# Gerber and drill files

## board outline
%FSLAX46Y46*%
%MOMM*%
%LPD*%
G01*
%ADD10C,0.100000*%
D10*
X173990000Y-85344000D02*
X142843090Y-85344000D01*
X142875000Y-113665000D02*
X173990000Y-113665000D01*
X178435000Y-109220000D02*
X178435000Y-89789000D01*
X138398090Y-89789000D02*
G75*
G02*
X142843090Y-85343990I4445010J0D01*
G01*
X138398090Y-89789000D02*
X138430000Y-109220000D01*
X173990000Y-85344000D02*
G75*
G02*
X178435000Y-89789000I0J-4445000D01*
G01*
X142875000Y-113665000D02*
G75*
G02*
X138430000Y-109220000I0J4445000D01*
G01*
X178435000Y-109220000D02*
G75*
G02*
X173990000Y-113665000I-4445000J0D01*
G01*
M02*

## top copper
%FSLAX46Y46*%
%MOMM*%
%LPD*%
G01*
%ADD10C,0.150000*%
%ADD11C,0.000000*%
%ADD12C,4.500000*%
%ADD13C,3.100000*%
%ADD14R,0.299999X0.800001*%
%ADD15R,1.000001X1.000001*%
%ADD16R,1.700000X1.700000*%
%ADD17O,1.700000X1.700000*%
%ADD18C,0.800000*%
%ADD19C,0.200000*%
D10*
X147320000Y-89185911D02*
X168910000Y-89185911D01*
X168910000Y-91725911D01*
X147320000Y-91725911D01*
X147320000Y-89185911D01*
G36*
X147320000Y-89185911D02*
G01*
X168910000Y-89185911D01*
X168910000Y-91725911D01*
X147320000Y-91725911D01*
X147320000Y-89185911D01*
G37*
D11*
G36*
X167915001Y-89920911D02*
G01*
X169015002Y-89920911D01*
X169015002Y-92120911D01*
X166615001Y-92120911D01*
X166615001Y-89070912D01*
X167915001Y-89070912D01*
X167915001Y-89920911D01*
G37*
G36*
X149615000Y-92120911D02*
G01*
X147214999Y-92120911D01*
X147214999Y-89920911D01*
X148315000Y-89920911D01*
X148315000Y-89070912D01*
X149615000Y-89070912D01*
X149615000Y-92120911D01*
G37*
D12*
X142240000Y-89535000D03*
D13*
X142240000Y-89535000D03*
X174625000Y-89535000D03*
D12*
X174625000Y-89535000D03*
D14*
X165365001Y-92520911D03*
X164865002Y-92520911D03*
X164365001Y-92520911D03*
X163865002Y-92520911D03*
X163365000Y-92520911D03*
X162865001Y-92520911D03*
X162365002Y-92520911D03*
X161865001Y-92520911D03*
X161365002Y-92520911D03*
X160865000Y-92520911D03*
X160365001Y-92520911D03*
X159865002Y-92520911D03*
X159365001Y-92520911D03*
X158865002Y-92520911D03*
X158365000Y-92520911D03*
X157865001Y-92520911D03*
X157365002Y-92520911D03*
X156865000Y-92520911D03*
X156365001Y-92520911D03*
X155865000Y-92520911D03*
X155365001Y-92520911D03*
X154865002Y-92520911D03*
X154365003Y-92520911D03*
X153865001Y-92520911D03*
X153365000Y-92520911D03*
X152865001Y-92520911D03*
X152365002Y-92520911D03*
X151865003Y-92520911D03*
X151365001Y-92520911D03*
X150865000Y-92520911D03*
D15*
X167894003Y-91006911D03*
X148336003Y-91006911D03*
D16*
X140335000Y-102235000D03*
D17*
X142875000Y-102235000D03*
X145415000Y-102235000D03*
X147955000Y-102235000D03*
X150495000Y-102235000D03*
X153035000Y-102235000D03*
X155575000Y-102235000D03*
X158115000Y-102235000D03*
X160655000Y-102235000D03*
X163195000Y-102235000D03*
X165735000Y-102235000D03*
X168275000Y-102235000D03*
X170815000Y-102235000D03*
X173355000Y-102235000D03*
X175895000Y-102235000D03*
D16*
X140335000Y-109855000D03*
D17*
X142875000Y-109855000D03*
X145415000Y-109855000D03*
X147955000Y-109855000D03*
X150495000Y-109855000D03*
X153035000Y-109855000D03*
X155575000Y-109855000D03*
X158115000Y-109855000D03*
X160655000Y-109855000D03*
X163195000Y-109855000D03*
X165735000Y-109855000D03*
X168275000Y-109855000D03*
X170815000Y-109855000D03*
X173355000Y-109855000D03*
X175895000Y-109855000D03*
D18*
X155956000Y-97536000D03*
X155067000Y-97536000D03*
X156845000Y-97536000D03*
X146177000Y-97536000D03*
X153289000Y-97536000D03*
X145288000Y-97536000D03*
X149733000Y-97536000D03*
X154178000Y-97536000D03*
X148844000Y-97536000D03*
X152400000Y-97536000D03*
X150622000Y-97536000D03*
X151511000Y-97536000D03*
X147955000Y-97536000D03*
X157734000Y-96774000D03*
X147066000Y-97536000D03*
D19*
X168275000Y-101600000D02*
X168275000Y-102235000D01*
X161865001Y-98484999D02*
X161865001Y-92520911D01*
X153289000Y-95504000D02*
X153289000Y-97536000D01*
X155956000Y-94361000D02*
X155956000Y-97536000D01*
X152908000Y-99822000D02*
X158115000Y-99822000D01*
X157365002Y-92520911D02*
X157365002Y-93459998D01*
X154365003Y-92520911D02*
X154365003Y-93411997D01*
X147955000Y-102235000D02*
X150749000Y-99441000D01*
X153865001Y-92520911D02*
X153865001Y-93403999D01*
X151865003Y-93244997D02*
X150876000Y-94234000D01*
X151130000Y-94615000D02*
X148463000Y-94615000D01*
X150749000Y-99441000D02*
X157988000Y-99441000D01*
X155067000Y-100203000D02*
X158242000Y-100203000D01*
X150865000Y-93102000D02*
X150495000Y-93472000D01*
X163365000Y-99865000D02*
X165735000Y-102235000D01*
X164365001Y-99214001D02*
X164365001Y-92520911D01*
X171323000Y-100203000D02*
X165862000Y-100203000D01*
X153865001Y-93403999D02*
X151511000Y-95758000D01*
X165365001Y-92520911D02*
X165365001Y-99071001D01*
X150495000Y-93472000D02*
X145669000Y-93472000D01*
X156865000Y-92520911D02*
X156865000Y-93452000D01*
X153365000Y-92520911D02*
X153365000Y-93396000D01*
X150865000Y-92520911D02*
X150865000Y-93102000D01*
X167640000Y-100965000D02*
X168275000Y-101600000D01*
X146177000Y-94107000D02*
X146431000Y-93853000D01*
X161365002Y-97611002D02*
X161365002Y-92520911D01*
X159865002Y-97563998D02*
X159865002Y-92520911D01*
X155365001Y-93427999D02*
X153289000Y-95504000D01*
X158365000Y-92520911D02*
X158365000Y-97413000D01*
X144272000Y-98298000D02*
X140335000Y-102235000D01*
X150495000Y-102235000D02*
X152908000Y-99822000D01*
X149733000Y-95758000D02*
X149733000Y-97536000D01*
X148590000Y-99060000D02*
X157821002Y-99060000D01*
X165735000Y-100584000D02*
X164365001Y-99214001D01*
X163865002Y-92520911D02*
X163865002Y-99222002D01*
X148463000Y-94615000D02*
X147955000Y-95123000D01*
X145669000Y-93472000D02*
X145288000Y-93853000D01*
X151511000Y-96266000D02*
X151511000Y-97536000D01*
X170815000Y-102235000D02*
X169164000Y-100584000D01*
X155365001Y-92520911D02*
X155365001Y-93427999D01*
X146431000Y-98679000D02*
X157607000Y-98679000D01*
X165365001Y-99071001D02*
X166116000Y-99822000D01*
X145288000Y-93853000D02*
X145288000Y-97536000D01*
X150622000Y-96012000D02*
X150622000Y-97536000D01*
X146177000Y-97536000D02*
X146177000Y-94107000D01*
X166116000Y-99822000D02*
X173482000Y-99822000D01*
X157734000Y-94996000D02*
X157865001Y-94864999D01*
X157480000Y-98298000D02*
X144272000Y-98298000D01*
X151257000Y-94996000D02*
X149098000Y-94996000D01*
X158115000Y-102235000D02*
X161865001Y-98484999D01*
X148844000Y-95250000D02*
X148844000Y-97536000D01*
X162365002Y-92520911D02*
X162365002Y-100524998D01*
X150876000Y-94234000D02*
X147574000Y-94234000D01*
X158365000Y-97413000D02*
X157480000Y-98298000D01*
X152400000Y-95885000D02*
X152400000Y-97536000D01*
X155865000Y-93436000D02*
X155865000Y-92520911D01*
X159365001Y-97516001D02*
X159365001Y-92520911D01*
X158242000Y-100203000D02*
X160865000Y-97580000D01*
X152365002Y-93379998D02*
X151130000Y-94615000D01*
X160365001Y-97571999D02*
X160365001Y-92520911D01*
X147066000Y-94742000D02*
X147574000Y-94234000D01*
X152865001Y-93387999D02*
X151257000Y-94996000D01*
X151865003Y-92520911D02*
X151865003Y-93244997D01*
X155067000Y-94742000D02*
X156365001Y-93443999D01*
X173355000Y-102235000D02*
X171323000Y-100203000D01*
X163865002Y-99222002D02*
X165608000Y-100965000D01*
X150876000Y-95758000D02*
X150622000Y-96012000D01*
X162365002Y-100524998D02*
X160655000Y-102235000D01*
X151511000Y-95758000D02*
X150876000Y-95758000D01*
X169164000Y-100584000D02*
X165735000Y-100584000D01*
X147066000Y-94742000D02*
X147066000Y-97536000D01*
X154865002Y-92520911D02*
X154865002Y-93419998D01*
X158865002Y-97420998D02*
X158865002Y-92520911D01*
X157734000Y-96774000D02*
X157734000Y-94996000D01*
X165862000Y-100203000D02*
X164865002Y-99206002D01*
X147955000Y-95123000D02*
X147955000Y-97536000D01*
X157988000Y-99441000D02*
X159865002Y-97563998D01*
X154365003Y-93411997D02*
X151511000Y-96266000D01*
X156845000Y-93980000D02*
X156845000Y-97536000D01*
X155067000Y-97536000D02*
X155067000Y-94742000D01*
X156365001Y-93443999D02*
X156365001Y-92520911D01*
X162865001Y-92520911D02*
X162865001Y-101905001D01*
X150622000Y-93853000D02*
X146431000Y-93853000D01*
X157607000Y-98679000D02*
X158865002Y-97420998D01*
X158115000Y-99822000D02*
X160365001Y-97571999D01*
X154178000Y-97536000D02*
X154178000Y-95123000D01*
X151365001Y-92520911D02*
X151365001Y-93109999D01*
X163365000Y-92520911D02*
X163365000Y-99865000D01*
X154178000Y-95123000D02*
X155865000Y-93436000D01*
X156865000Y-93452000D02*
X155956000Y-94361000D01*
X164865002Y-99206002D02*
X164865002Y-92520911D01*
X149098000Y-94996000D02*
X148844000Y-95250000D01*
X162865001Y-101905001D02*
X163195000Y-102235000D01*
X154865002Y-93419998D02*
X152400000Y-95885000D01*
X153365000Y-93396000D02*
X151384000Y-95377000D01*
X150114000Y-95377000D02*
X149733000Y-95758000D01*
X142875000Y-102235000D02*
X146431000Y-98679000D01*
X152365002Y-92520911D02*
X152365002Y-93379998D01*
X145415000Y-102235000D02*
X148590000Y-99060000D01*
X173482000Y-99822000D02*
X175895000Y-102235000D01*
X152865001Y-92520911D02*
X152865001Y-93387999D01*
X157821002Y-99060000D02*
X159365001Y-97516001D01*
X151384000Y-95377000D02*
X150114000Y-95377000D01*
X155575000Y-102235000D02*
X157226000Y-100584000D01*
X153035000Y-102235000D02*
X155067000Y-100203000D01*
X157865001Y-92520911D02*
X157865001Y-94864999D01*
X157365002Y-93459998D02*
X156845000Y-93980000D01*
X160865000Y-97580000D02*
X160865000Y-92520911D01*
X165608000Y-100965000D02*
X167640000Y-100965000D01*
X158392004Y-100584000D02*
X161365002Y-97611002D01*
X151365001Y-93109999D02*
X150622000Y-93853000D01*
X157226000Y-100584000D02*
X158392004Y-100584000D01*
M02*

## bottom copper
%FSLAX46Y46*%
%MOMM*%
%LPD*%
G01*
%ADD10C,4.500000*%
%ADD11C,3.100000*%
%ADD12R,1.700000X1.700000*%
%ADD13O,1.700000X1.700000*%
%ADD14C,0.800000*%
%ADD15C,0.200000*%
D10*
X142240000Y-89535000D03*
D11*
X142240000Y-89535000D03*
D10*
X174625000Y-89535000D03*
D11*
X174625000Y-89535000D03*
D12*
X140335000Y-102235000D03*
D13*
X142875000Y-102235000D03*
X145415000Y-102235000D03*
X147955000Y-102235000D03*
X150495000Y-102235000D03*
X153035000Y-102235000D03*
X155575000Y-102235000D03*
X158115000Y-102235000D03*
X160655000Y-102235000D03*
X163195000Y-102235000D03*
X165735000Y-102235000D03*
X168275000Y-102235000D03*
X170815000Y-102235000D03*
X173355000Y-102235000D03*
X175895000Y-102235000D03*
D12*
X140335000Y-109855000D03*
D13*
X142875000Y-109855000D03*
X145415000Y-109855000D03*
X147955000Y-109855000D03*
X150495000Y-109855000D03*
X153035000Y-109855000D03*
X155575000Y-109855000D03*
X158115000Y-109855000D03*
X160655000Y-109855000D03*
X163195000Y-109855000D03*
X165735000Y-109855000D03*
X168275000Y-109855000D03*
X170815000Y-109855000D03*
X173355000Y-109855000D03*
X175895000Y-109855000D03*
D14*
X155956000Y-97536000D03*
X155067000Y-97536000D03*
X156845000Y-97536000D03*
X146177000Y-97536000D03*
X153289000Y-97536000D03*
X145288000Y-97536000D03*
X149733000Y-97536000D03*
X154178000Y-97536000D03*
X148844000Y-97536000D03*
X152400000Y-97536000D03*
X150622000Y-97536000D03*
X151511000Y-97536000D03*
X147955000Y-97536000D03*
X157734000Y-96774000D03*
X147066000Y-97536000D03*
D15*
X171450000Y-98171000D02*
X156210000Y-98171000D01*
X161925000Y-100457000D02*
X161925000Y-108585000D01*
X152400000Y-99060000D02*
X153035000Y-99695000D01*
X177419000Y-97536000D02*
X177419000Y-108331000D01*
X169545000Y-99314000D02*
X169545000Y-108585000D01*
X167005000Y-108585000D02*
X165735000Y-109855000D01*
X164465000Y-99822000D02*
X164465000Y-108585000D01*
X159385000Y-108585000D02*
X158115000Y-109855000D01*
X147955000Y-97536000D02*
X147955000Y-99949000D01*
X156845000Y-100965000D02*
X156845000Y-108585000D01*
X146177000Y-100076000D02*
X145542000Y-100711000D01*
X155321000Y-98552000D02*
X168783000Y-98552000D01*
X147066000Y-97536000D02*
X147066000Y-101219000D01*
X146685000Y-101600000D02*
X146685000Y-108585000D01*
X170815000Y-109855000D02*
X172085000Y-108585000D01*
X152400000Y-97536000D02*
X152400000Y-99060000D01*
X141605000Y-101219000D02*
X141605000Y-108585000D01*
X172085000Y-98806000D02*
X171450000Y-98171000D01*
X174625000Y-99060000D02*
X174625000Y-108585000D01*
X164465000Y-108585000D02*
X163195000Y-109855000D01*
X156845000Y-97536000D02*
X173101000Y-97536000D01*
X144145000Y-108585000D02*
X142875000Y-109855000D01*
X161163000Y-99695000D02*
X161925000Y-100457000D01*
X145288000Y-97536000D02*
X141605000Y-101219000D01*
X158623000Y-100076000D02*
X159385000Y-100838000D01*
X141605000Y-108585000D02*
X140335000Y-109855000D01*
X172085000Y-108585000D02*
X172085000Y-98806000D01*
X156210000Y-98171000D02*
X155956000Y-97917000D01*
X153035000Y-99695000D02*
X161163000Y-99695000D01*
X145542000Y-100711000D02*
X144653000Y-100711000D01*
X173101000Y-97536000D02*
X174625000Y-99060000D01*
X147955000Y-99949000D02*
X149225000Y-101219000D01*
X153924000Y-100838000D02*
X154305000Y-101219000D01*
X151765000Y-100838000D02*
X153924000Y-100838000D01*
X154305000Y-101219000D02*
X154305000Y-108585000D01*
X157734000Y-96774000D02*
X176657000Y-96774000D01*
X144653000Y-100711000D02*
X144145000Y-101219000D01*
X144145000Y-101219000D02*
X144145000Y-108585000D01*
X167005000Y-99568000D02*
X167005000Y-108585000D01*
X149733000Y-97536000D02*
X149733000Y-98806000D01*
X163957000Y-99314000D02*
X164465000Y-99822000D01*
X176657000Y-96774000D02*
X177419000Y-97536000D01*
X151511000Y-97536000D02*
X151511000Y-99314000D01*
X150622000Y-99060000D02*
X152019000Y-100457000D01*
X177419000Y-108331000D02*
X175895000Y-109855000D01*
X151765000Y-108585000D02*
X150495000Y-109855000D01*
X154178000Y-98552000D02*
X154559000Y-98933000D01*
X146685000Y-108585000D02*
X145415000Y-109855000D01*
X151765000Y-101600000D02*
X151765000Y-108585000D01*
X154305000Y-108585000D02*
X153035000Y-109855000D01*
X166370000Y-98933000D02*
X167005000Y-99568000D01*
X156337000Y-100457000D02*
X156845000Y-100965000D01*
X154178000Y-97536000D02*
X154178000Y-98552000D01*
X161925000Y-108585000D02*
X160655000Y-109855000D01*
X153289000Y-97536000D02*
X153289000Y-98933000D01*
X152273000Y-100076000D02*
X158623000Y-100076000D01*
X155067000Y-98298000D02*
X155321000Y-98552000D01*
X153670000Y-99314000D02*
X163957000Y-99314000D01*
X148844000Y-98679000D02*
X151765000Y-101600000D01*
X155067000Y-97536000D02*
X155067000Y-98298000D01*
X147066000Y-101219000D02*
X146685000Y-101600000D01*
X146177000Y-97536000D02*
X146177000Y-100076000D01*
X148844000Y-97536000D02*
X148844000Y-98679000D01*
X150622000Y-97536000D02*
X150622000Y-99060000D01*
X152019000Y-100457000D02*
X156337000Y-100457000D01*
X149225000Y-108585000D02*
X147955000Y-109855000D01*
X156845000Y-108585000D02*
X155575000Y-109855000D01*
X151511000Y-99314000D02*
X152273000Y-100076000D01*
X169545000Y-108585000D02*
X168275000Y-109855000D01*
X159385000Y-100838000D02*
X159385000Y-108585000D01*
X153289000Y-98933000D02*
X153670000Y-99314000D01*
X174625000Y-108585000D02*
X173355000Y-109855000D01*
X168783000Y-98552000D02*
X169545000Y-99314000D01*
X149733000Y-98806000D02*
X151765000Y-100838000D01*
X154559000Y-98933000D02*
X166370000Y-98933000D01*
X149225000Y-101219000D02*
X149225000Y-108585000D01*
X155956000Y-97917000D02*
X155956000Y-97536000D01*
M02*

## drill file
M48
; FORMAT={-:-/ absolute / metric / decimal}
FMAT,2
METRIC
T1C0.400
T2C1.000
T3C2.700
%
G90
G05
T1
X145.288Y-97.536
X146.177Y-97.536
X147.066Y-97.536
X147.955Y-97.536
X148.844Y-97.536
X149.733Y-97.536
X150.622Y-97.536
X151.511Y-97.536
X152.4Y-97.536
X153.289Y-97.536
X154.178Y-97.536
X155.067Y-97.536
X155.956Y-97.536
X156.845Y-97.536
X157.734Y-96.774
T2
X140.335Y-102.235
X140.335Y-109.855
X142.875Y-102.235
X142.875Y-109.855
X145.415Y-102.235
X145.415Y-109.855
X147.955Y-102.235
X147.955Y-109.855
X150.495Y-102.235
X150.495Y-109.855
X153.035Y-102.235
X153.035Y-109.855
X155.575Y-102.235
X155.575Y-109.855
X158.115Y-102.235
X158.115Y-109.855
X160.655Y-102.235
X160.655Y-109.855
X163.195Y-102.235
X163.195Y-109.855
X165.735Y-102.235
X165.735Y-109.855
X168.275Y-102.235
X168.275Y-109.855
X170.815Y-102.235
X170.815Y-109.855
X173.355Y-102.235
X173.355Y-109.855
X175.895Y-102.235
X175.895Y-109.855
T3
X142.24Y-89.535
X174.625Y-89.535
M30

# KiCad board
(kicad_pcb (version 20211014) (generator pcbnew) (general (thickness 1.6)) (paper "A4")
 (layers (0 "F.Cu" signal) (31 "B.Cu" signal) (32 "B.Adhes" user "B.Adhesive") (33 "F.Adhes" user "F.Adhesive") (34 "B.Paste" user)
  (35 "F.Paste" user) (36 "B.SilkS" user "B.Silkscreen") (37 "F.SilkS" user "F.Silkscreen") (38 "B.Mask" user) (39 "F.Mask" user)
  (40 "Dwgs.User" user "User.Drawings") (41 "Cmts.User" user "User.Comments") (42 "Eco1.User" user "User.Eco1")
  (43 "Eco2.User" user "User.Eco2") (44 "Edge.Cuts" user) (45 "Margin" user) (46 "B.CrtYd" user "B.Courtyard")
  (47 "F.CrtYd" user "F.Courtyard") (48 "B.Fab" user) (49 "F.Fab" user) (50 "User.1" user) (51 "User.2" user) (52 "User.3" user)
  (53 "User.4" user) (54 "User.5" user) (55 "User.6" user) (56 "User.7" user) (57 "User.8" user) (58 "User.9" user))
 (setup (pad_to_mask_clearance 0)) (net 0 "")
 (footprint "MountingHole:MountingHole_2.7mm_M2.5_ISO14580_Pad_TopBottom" (layer "F.Cu") (at 142.24 89.535)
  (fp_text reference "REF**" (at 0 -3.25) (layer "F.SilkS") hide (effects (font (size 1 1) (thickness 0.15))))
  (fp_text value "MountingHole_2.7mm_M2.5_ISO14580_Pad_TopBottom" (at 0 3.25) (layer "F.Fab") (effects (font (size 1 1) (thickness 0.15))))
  (pad "1" connect circle (at 0 0) (size 4.5 4.5) (layers "B.Cu" "B.Mask"))
  (pad "1" connect circle (at 0 0) (size 4.5 4.5) (layers "F.Cu" "F.Mask"))
  (pad "1" thru_hole circle (at 0 0) (size 3.1 3.1) (drill 2.7) (layers *.Cu *.Mask)))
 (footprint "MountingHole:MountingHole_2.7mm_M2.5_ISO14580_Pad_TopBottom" (layer "F.Cu") (at 174.625 89.535)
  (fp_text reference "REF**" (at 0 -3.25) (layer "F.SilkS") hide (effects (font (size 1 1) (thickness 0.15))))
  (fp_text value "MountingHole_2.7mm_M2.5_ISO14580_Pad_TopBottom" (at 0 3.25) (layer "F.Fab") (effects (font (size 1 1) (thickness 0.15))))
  (pad "1" connect circle (at 0 0) (size 4.5 4.5) (layers "B.Cu" "B.Mask"))
  (pad "1" thru_hole circle (at 0 0) (size 3.1 3.1) (drill 2.7) (layers *.Cu *.Mask))
  (pad "1" connect circle (at 0 0) (size 4.5 4.5) (layers "F.Cu" "F.Mask")))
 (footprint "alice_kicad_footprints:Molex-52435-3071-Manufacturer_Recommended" (layer "F.Cu") (at 158.115003 91.758908 180)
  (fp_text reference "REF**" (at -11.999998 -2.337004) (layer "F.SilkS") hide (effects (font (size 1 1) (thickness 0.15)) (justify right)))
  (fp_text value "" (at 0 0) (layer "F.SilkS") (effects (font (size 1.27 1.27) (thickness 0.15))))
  (fp_poly
   (pts (xy -8.499998 -0.362003) (xy -10.899999 -0.362003) (xy -10.899999 1.837997) (xy -9.799998 1.837997) (xy -9.799998 2.687996)
    (xy -8.499998 2.687996))
   (layer "F.Cu") (width 0) (fill solid))
  (fp_poly
   (pts (xy 8.500003 -0.362003) (xy 10.900004 -0.362003) (xy 10.900004 1.837997) (xy 9.800003 1.837997) (xy 9.800003 2.687996)
    (xy 8.500003 2.687996))
   (layer "F.Cu") (width 0) (fill solid))
  (pad "1" smd rect locked (at -7.249998 -0.762003) (size 0.299999 0.800001) (layers "F.Cu" "F.Paste" "F.Mask"))
  (pad "2" smd rect locked (at -6.749999 -0.762003) (size 0.299999 0.800001) (layers "F.Cu" "F.Paste" "F.Mask"))
  (pad "3" smd rect locked (at -6.249998 -0.762003) (size 0.299999 0.800001) (layers "F.Cu" "F.Paste" "F.Mask"))
  (pad "4" smd rect locked (at -5.749999 -0.762003) (size 0.299999 0.800001) (layers "F.Cu" "F.Paste" "F.Mask"))
  (pad "5" smd rect locked (at -5.249997 -0.762003) (size 0.299999 0.800001) (layers "F.Cu" "F.Paste" "F.Mask"))
  (pad "6" smd rect locked (at -4.749998 -0.762003) (size 0.299999 0.800001) (layers "F.Cu" "F.Paste" "F.Mask"))
  (pad "7" smd rect locked (at -4.249999 -0.762003) (size 0.299999 0.800001) (layers "F.Cu" "F.Paste" "F.Mask"))
  (pad "8" smd rect locked (at -3.749998 -0.762003) (size 0.299999 0.800001) (layers "F.Cu" "F.Paste" "F.Mask"))
  (pad "9" smd rect locked (at -3.249999 -0.762003) (size 0.299999 0.800001) (layers "F.Cu" "F.Paste" "F.Mask"))
  (pad "10" smd rect locked (at -2.749997 -0.762003) (size 0.299999 0.800001) (layers "F.Cu" "F.Paste" "F.Mask"))
  (pad "11" smd rect locked (at -2.249998 -0.762003) (size 0.299999 0.800001) (layers "F.Cu" "F.Paste" "F.Mask"))
  (pad "12" smd rect locked (at -1.749999 -0.762003) (size 0.299999 0.800001) (layers "F.Cu" "F.Paste" "F.Mask"))
  (pad "13" smd rect locked (at -1.249998 -0.762003) (size 0.299999 0.800001) (layers "F.Cu" "F.Paste" "F.Mask"))
  (pad "14" smd rect locked (at -0.749999 -0.762003) (size 0.299999 0.800001) (layers "F.Cu" "F.Paste" "F.Mask"))
  (pad "15" smd rect locked (at -0.249997 -0.762003) (size 0.299999 0.800001) (layers "F.Cu" "F.Paste" "F.Mask"))
  (pad "16" smd rect locked (at 0.250002 -0.762003) (size 0.299999 0.800001) (layers "F.Cu" "F.Paste" "F.Mask"))
  (pad "17" smd rect locked (at 0.750001 -0.762003) (size 0.299999 0.800001) (layers "F.Cu" "F.Paste" "F.Mask"))
  (pad "18" smd rect locked (at 1.250003 -0.762003) (size 0.299999 0.800001) (layers "F.Cu" "F.Paste" "F.Mask"))
  (pad "19" smd rect locked (at 1.750002 -0.762003) (size 0.299999 0.800001) (layers "F.Cu" "F.Paste" "F.Mask"))
  (pad "20" smd rect locked (at 2.250003 -0.762003) (size 0.299999 0.800001) (layers "F.Cu" "F.Paste" "F.Mask"))
  (pad "21" smd rect locked (at 2.750002 -0.762003) (size 0.299999 0.800001) (layers "F.Cu" "F.Paste" "F.Mask"))
  (pad "22" smd rect locked (at 3.250001 -0.762003) (size 0.299999 0.800001) (layers "F.Cu" "F.Paste" "F.Mask"))
  (pad "23" smd rect locked (at 3.75 -0.762003) (size 0.299999 0.800001) (layers "F.Cu" "F.Paste" "F.Mask"))
  (pad "24" smd rect locked (at 4.250002 -0.762003) (size 0.299999 0.800001) (layers "F.Cu" "F.Paste" "F.Mask"))
  (pad "25" smd rect locked (at 4.750003 -0.762003) (size 0.299999 0.800001) (layers "F.Cu" "F.Paste" "F.Mask"))
  (pad "26" smd rect locked (at 5.250002 -0.762003) (size 0.299999 0.800001) (layers "F.Cu" "F.Paste" "F.Mask"))
  (pad "27" smd rect locked (at 5.750001 -0.762003) (size 0.299999 0.800001) (layers "F.Cu" "F.Paste" "F.Mask"))
  (pad "28" smd rect locked (at 6.25 -0.762003) (size 0.299999 0.800001) (layers "F.Cu" "F.Paste" "F.Mask"))
  (pad "29" smd rect locked (at 6.750002 -0.762003) (size 0.299999 0.800001) (layers "F.Cu" "F.Paste" "F.Mask"))
  (pad "30" smd rect locked (at 7.250003 -0.762003) (size 0.299999 0.800001) (layers "F.Cu" "F.Paste" "F.Mask"))
  (pad "MP1" smd rect locked (at -9.779 0.751997) (size 1.000001 1.000001) (layers "F.Cu" "F.Paste" "F.Mask"))
  (pad "MP2" smd rect locked (at 9.779 0.751997) (size 1.000001 1.000001) (layers "F.Cu" "F.Paste" "F.Mask")))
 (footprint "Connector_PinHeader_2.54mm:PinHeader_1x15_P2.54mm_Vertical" (layer "F.Cu") (at 140.335 102.235 90)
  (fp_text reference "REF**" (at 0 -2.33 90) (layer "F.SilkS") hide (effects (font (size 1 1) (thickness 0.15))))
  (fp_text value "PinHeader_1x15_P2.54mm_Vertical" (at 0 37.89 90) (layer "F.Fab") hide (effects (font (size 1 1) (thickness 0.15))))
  (pad "1" thru_hole rect (at 0 0 90) (size 1.7 1.7) (drill 1) (layers *.Cu *.Mask))
  (pad "2" thru_hole oval (at 0 2.54 90) (size 1.7 1.7) (drill 1) (layers *.Cu *.Mask))
  (pad "3" thru_hole oval (at 0 5.08 90) (size 1.7 1.7) (drill 1) (layers *.Cu *.Mask))
  (pad "4" thru_hole oval (at 0 7.62 90) (size 1.7 1.7) (drill 1) (layers *.Cu *.Mask))
  (pad "5" thru_hole oval (at 0 10.16 90) (size 1.7 1.7) (drill 1) (layers *.Cu *.Mask))
  (pad "6" thru_hole oval (at 0 12.7 90) (size 1.7 1.7) (drill 1) (layers *.Cu *.Mask))
  (pad "7" thru_hole oval (at 0 15.24 90) (size 1.7 1.7) (drill 1) (layers *.Cu *.Mask))
  (pad "8" thru_hole oval (at 0 17.78 90) (size 1.7 1.7) (drill 1) (layers *.Cu *.Mask))
  (pad "9" thru_hole oval (at 0 20.32 90) (size 1.7 1.7) (drill 1) (layers *.Cu *.Mask))
  (pad "10" thru_hole oval (at 0 22.86 90) (size 1.7 1.7) (drill 1) (layers *.Cu *.Mask))
  (pad "11" thru_hole oval (at 0 25.4 90) (size 1.7 1.7) (drill 1) (layers *.Cu *.Mask))
  (pad "12" thru_hole oval (at 0 27.94 90) (size 1.7 1.7) (drill 1) (layers *.Cu *.Mask))
  (pad "13" thru_hole oval (at 0 30.48 90) (size 1.7 1.7) (drill 1) (layers *.Cu *.Mask))
  (pad "14" thru_hole oval (at 0 33.02 90) (size 1.7 1.7) (drill 1) (layers *.Cu *.Mask))
  (pad "15" thru_hole oval (at 0 35.56 90) (size 1.7 1.7) (drill 1) (layers *.Cu *.Mask)))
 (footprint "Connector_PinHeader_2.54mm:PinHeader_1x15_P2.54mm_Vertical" (layer "F.Cu") (at 140.335 109.855 90)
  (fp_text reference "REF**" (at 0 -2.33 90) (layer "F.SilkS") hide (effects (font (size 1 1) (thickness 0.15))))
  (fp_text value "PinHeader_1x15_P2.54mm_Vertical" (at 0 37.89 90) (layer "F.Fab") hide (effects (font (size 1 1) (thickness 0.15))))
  (pad "1" thru_hole rect (at 0 0 90) (size 1.7 1.7) (drill 1) (layers *.Cu *.Mask))
  (pad "2" thru_hole oval (at 0 2.54 90) (size 1.7 1.7) (drill 1) (layers *.Cu *.Mask))
  (pad "3" thru_hole oval (at 0 5.08 90) (size 1.7 1.7) (drill 1) (layers *.Cu *.Mask))
  (pad "4" thru_hole oval (at 0 7.62 90) (size 1.7 1.7) (drill 1) (layers *.Cu *.Mask))
  (pad "5" thru_hole oval (at 0 10.16 90) (size 1.7 1.7) (drill 1) (layers *.Cu *.Mask))
  (pad "6" thru_hole oval (at 0 12.7 90) (size 1.7 1.7) (drill 1) (layers *.Cu *.Mask))
  (pad "7" thru_hole oval (at 0 15.24 90) (size 1.7 1.7) (drill 1) (layers *.Cu *.Mask))
  (pad "8" thru_hole oval (at 0 17.78 90) (size 1.7 1.7) (drill 1) (layers *.Cu *.Mask))
  (pad "9" thru_hole oval (at 0 20.32 90) (size 1.7 1.7) (drill 1) (layers *.Cu *.Mask))
  (pad "10" thru_hole oval (at 0 22.86 90) (size 1.7 1.7) (drill 1) (layers *.Cu *.Mask))
  (pad "11" thru_hole oval (at 0 25.4 90) (size 1.7 1.7) (drill 1) (layers *.Cu *.Mask))
  (pad "12" thru_hole oval (at 0 27.94 90) (size 1.7 1.7) (drill 1) (layers *.Cu *.Mask))
  (pad "13" thru_hole oval (at 0 30.48 90) (size 1.7 1.7) (drill 1) (layers *.Cu *.Mask))
  (pad "14" thru_hole oval (at 0 33.02 90) (size 1.7 1.7) (drill 1) (layers *.Cu *.Mask))
  (pad "15" thru_hole oval (at 0 35.56 90) (size 1.7 1.7) (drill 1) (layers *.Cu *.Mask)))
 (gr_rect (start 147.32 91.725911) (end 168.91 89.185911) (layer "F.Cu") (width 0.15) (fill solid))
 (gr_line (start 173.99 85.344) (end 142.84309 85.344) (layer "Edge.Cuts") (width 0.1))
 (gr_line (start 142.875 113.665) (end 173.99 113.665) (layer "Edge.Cuts") (width 0.1))
 (gr_line (start 178.435 109.22) (end 178.435 89.789) (layer "Edge.Cuts") (width 0.1))
 (gr_arc (start 138.39809 89.789) (mid 139.7 86.64591) (end 142.84309 85.344) (layer "Edge.Cuts") (width 0.1))
 (gr_line (start 138.39809 89.789) (end 138.43 109.22) (layer "Edge.Cuts") (width 0.1))
 (gr_arc (start 173.99 85.344) (mid 177.13309 86.64591) (end 178.435 89.789) (layer "Edge.Cuts") (width 0.1))
 (gr_arc (start 142.875 113.665) (mid 139.73191 112.36309) (end 138.43 109.22) (layer "Edge.Cuts") (width 0.1))
 (gr_arc (start 178.435 109.22) (mid 177.13309 112.36309) (end 173.99 113.665) (layer "Edge.Cuts") (width 0.1))
 (segment (start 168.275 101.6) (end 168.275 102.235) (width 0.2) (layer "F.Cu") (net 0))
 (segment (start 161.865001 98.484999) (end 161.865001 92.520911) (width 0.2) (layer "F.Cu") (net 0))
 (segment (start 153.289 95.504) (end 153.289 97.536) (width 0.2) (layer "F.Cu") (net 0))
 (segment (start 155.956 94.361) (end 155.956 97.536) (width 0.2) (layer "F.Cu") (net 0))
 (segment (start 152.908 99.822) (end 158.115 99.822) (width 0.2) (layer "F.Cu") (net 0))
 (segment (start 157.365002 92.520911) (end 157.365002 93.459998) (width 0.2) (layer "F.Cu") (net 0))
 (segment (start 154.365003 92.520911) (end 154.365003 93.411997) (width 0.2) (layer "F.Cu") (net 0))
 (segment (start 147.955 102.235) (end 150.749 99.441) (width 0.2) (layer "F.Cu") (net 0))
 (segment (start 153.865001 92.520911) (end 153.865001 93.403999) (width 0.2) (layer "F.Cu") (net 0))
 (segment (start 151.865003 93.244997) (end 150.876 94.234) (width 0.2) (layer "F.Cu") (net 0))
 (segment (start 151.13 94.615) (end 148.463 94.615) (width 0.2) (layer "F.Cu") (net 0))
 (segment (start 150.749 99.441) (end 157.988 99.441) (width 0.2) (layer "F.Cu") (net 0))
 (segment (start 155.067 100.203) (end 158.242 100.203) (width 0.2) (layer "F.Cu") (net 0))
 (segment (start 150.865 93.102) (end 150.495 93.472) (width 0.2) (layer "F.Cu") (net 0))
 (segment (start 163.365 99.865) (end 165.735 102.235) (width 0.2) (layer "F.Cu") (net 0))
 (segment (start 164.365001 99.214001) (end 164.365001 92.520911) (width 0.2) (layer "F.Cu") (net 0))
 (segment (start 171.323 100.203) (end 165.862 100.203) (width 0.2) (layer "F.Cu") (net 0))
 (segment (start 153.865001 93.403999) (end 151.511 95.758) (width 0.2) (layer "F.Cu") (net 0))
 (segment (start 165.365001 92.520911) (end 165.365001 99.071001) (width 0.2) (layer "F.Cu") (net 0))
 (segment (start 150.495 93.472) (end 145.669 93.472) (width 0.2) (layer "F.Cu") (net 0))
 (segment (start 156.865 92.520911) (end 156.865 93.452) (width 0.2) (layer "F.Cu") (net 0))
 (segment (start 153.365 92.520911) (end 153.365 93.396) (width 0.2) (layer "F.Cu") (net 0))
 (segment (start 150.865 92.520911) (end 150.865 93.102) (width 0.2) (layer "F.Cu") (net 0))
 (segment (start 167.64 100.965) (end 168.275 101.6) (width 0.2) (layer "F.Cu") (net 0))
 (segment (start 146.177 94.107) (end 146.431 93.853) (width 0.2) (layer "F.Cu") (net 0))
 (segment (start 161.365002 97.611002) (end 161.365002 92.520911) (width 0.2) (layer "F.Cu") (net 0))
 (segment (start 159.865002 97.563998) (end 159.865002 92.520911) (width 0.2) (layer "F.Cu") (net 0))
 (segment (start 155.365001 93.427999) (end 153.289 95.504) (width 0.2) (layer "F.Cu") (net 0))
 (segment (start 158.365 92.520911) (end 158.365 97.413) (width 0.2) (layer "F.Cu") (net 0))
 (segment (start 144.272 98.298) (end 140.335 102.235) (width 0.2) (layer "F.Cu") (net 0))
 (segment (start 150.495 102.235) (end 152.908 99.822) (width 0.2) (layer "F.Cu") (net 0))
 (segment (start 149.733 95.758) (end 149.733 97.536) (width 0.2) (layer "F.Cu") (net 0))
 (segment (start 148.59 99.06) (end 157.821002 99.06) (width 0.2) (layer "F.Cu") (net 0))
 (segment (start 165.735 100.584) (end 164.365001 99.214001) (width 0.2) (layer "F.Cu") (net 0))
 (segment (start 163.865002 92.520911) (end 163.865002 99.222002) (width 0.2) (layer "F.Cu") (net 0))
 (segment (start 148.463 94.615) (end 147.955 95.123) (width 0.2) (layer "F.Cu") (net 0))
 (segment (start 145.669 93.472) (end 145.288 93.853) (width 0.2) (layer "F.Cu") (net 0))
 (segment (start 151.511 96.266) (end 151.511 97.536) (width 0.2) (layer "F.Cu") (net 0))
 (segment (start 170.815 102.235) (end 169.164 100.584) (width 0.2) (layer "F.Cu") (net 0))
 (segment (start 155.365001 92.520911) (end 155.365001 93.427999) (width 0.2) (layer "F.Cu") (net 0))
 (segment (start 146.431 98.679) (end 157.607 98.679) (width 0.2) (layer "F.Cu") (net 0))
 (segment (start 165.365001 99.071001) (end 166.116 99.822) (width 0.2) (layer "F.Cu") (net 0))
 (segment (start 145.288 93.853) (end 145.288 97.536) (width 0.2) (layer "F.Cu") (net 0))
 (segment (start 150.622 96.012) (end 150.622 97.536) (width 0.2) (layer "F.Cu") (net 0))
 (segment (start 146.177 97.536) (end 146.177 94.107) (width 0.2) (layer "F.Cu") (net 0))
 (segment (start 166.116 99.822) (end 173.482 99.822) (width 0.2) (layer "F.Cu") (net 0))
 (segment (start 157.734 94.996) (end 157.865001 94.864999) (width 0.2) (layer "F.Cu") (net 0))
 (segment (start 157.48 98.298) (end 144.272 98.298) (width 0.2) (layer "F.Cu") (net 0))
 (segment (start 151.257 94.996) (end 149.098 94.996) (width 0.2) (layer "F.Cu") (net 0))
 (segment (start 158.115 102.235) (end 161.865001 98.484999) (width 0.2) (layer "F.Cu") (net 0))
 (segment (start 148.844 95.25) (end 148.844 97.536) (width 0.2) (layer "F.Cu") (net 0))
 (segment (start 162.365002 92.520911) (end 162.365002 100.524998) (width 0.2) (layer "F.Cu") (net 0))
 (segment (start 150.876 94.234) (end 147.574 94.234) (width 0.2) (layer "F.Cu") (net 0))
 (segment (start 158.365 97.413) (end 157.48 98.298) (width 0.2) (layer "F.Cu") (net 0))
 (segment (start 152.4 95.885) (end 152.4 97.536) (width 0.2) (layer "F.Cu") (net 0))
 (segment (start 155.865 93.436) (end 155.865 92.520911) (width 0.2) (layer "F.Cu") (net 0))
 (segment (start 159.365001 97.516001) (end 159.365001 92.520911) (width 0.2) (layer "F.Cu") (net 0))
 (segment (start 158.242 100.203) (end 160.865 97.58) (width 0.2) (layer "F.Cu") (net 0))
 (segment (start 152.365002 93.379998) (end 151.13 94.615) (width 0.2) (layer "F.Cu") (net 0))
 (segment (start 160.365001 97.571999) (end 160.365001 92.520911) (width 0.2) (layer "F.Cu") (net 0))
 (segment (start 147.066 94.742) (end 147.574 94.234) (width 0.2) (layer "F.Cu") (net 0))
 (segment (start 152.865001 93.387999) (end 151.257 94.996) (width 0.2) (layer "F.Cu") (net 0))
 (segment (start 151.865003 92.520911) (end 151.865003 93.244997) (width 0.2) (layer "F.Cu") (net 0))
 (segment (start 155.067 94.742) (end 156.365001 93.443999) (width 0.2) (layer "F.Cu") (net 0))
 (segment (start 173.355 102.235) (end 171.323 100.203) (width 0.2) (layer "F.Cu") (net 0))
 (segment (start 163.865002 99.222002) (end 165.608 100.965) (width 0.2) (layer "F.Cu") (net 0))
 (segment (start 150.876 95.758) (end 150.622 96.012) (width 0.2) (layer "F.Cu") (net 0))
 (segment (start 162.365002 100.524998) (end 160.655 102.235) (width 0.2) (layer "F.Cu") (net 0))
 (segment (start 151.511 95.758) (end 150.876 95.758) (width 0.2) (layer "F.Cu") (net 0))
 (segment (start 169.164 100.584) (end 165.735 100.584) (width 0.2) (layer "F.Cu") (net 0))
 (segment (start 147.066 94.742) (end 147.066 97.536) (width 0.2) (layer "F.Cu") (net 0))
 (segment (start 154.865002 92.520911) (end 154.865002 93.419998) (width 0.2) (layer "F.Cu") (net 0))
 (segment (start 158.865002 97.420998) (end 158.865002 92.520911) (width 0.2) (layer "F.Cu") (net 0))
 (segment (start 157.734 96.774) (end 157.734 94.996) (width 0.2) (layer "F.Cu") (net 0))
 (segment (start 165.862 100.203) (end 164.865002 99.206002) (width 0.2) (layer "F.Cu") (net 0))
 (segment (start 147.955 95.123) (end 147.955 97.536) (width 0.2) (layer "F.Cu") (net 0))
 (segment (start 157.988 99.441) (end 159.865002 97.563998) (width 0.2) (layer "F.Cu") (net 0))
 (segment (start 154.365003 93.411997) (end 151.511 96.266) (width 0.2) (layer "F.Cu") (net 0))
 (segment (start 156.845 93.98) (end 156.845 97.536) (width 0.2) (layer "F.Cu") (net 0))
 (segment (start 155.067 97.536) (end 155.067 94.742) (width 0.2) (layer "F.Cu") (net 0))
 (segment (start 156.365001 93.443999) (end 156.365001 92.520911) (width 0.2) (layer "F.Cu") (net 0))
 (segment (start 162.865001 92.520911) (end 162.865001 101.905001) (width 0.2) (layer "F.Cu") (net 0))
 (segment (start 150.622 93.853) (end 146.431 93.853) (width 0.2) (layer "F.Cu") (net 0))
 (segment (start 157.607 98.679) (end 158.865002 97.420998) (width 0.2) (layer "F.Cu") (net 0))
 (segment (start 158.115 99.822) (end 160.365001 97.571999) (width 0.2) (layer "F.Cu") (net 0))
 (segment (start 154.178 97.536) (end 154.178 95.123) (width 0.2) (layer "F.Cu") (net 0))
 (segment (start 151.365001 92.520911) (end 151.365001 93.109999) (width 0.2) (layer "F.Cu") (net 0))
 (segment (start 163.365 92.520911) (end 163.365 99.865) (width 0.2) (layer "F.Cu") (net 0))
 (segment (start 154.178 95.123) (end 155.865 93.436) (width 0.2) (layer "F.Cu") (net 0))
 (segment (start 156.865 93.452) (end 155.956 94.361) (width 0.2) (layer "F.Cu") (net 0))
 (segment (start 164.865002 99.206002) (end 164.865002 92.520911) (width 0.2) (layer "F.Cu") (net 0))
 (segment (start 149.098 94.996) (end 148.844 95.25) (width 0.2) (layer "F.Cu") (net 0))
 (segment (start 162.865001 101.905001) (end 163.195 102.235) (width 0.2) (layer "F.Cu") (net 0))
 (segment (start 154.865002 93.419998) (end 152.4 95.885) (width 0.2) (layer "F.Cu") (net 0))
 (segment (start 153.365 93.396) (end 151.384 95.377) (width 0.2) (layer "F.Cu") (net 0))
 (segment (start 150.114 95.377) (end 149.733 95.758) (width 0.2) (layer "F.Cu") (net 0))
 (segment (start 142.875 102.235) (end 146.431 98.679) (width 0.2) (layer "F.Cu") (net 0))
 (segment (start 152.365002 92.520911) (end 152.365002 93.379998) (width 0.2) (layer "F.Cu") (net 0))
 (segment (start 145.415 102.235) (end 148.59 99.06) (width 0.2) (layer "F.Cu") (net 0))
 (segment (start 173.482 99.822) (end 175.895 102.235) (width 0.2) (layer "F.Cu") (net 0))
 (segment (start 152.865001 92.520911) (end 152.865001 93.387999) (width 0.2) (layer "F.Cu") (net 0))
 (segment (start 157.821002 99.06) (end 159.365001 97.516001) (width 0.2) (layer "F.Cu") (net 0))
 (segment (start 151.384 95.377) (end 150.114 95.377) (width 0.2) (layer "F.Cu") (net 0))
 (segment (start 155.575 102.235) (end 157.226 100.584) (width 0.2) (layer "F.Cu") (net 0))
 (segment (start 153.035 102.235) (end 155.067 100.203) (width 0.2) (layer "F.Cu") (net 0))
 (segment (start 157.865001 92.520911) (end 157.865001 94.864999) (width 0.2) (layer "F.Cu") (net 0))
 (segment (start 157.365002 93.459998) (end 156.845 93.98) (width 0.2) (layer "F.Cu") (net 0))
 (segment (start 160.865 97.58) (end 160.865 92.520911) (width 0.2) (layer "F.Cu") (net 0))
 (segment (start 165.608 100.965) (end 167.64 100.965) (width 0.2) (layer "F.Cu") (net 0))
 (segment (start 158.392004 100.584) (end 161.365002 97.611002) (width 0.2) (layer "F.Cu") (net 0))
 (segment (start 151.365001 93.109999) (end 150.622 93.853) (width 0.2) (layer "F.Cu") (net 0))
 (segment (start 157.226 100.584) (end 158.392004 100.584) (width 0.2) (layer "F.Cu") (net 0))
 (via (at 155.956 97.536) (size 0.8) (drill 0.4) (layers "F.Cu" "B.Cu") (free) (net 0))
 (via (at 155.067 97.536) (size 0.8) (drill 0.4) (layers "F.Cu" "B.Cu") (free) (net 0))
 (via (at 156.845 97.536) (size 0.8) (drill 0.4) (layers "F.Cu" "B.Cu") (free) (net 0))
 (via (at 146.177 97.536) (size 0.8) (drill 0.4) (layers "F.Cu" "B.Cu") (free) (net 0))
 (via (at 153.289 97.536) (size 0.8) (drill 0.4) (layers "F.Cu" "B.Cu") (free) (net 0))
 (via (at 145.288 97.536) (size 0.8) (drill 0.4) (layers "F.Cu" "B.Cu") (free) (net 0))
 (via (at 149.733 97.536) (size 0.8) (drill 0.4) (layers "F.Cu" "B.Cu") (free) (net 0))
 (via (at 154.178 97.536) (size 0.8) (drill 0.4) (layers "F.Cu" "B.Cu") (free) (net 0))
 (via (at 148.844 97.536) (size 0.8) (drill 0.4) (layers "F.Cu" "B.Cu") (free) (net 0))
 (via (at 152.4 97.536) (size 0.8) (drill 0.4) (layers "F.Cu" "B.Cu") (free) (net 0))
 (via (at 150.622 97.536) (size 0.8) (drill 0.4) (layers "F.Cu" "B.Cu") (free) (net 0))
 (via (at 151.511 97.536) (size 0.8) (drill 0.4) (layers "F.Cu" "B.Cu") (free) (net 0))
 (via (at 147.955 97.536) (size 0.8) (drill 0.4) (layers "F.Cu" "B.Cu") (free) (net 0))
 (via (at 157.734 96.774) (size 0.8) (drill 0.4) (layers "F.Cu" "B.Cu") (free) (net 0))
 (via (at 147.066 97.536) (size 0.8) (drill 0.4) (layers "F.Cu" "B.Cu") (free) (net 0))
 (segment (start 171.45 98.171) (end 156.21 98.171) (width 0.2) (layer "B.Cu") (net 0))
 (segment (start 161.925 100.457) (end 161.925 108.585) (width 0.2) (layer "B.Cu") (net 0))
 (segment (start 152.4 99.06) (end 153.035 99.695) (width 0.2) (layer "B.Cu") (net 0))
 (segment (start 177.419 97.536) (end 177.419 108.331) (width 0.2) (layer "B.Cu") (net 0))
 (segment (start 169.545 99.314) (end 169.545 108.585) (width 0.2) (layer "B.Cu") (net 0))
 (segment (start 167.005 108.585) (end 165.735 109.855) (width 0.2) (layer "B.Cu") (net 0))
 (segment (start 164.465 99.822) (end 164.465 108.585) (width 0.2) (layer "B.Cu") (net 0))
 (segment (start 159.385 108.585) (end 158.115 109.855) (width 0.2) (layer "B.Cu") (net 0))
 (segment (start 147.955 97.536) (end 147.955 99.949) (width 0.2) (layer "B.Cu") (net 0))
 (segment (start 156.845 100.965) (end 156.845 108.585) (width 0.2) (layer "B.Cu") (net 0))
 (segment (start 146.177 100.076) (end 145.542 100.711) (width 0.2) (layer "B.Cu") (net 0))
 (segment (start 155.321 98.552) (end 168.783 98.552) (width 0.2) (layer "B.Cu") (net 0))
 (segment (start 147.066 97.536) (end 147.066 101.219) (width 0.2) (layer "B.Cu") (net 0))
 (segment (start 146.685 101.6) (end 146.685 108.585) (width 0.2) (layer "B.Cu") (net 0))
 (segment (start 170.815 109.855) (end 172.085 108.585) (width 0.2) (layer "B.Cu") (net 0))
 (segment (start 152.4 97.536) (end 152.4 99.06) (width 0.2) (layer "B.Cu") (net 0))
 (segment (start 141.605 101.219) (end 141.605 108.585) (width 0.2) (layer "B.Cu") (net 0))
 (segment (start 172.085 98.806) (end 171.45 98.171) (width 0.2) (layer "B.Cu") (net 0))
 (segment (start 174.625 99.06) (end 174.625 108.585) (width 0.2) (layer "B.Cu") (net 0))
 (segment (start 164.465 108.585) (end 163.195 109.855) (width 0.2) (layer "B.Cu") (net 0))
 (segment (start 156.845 97.536) (end 173.101 97.536) (width 0.2) (layer "B.Cu") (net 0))
 (segment (start 144.145 108.585) (end 142.875 109.855) (width 0.2) (layer "B.Cu") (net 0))
 (segment (start 161.163 99.695) (end 161.925 100.457) (width 0.2) (layer "B.Cu") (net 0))
 (segment (start 145.288 97.536) (end 141.605 101.219) (width 0.2) (layer "B.Cu") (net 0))
 (segment (start 158.623 100.076) (end 159.385 100.838) (width 0.2) (layer "B.Cu") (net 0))
 (segment (start 141.605 108.585) (end 140.335 109.855) (width 0.2) (layer "B.Cu") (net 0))
 (segment (start 172.085 108.585) (end 172.085 98.806) (width 0.2) (layer "B.Cu") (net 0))
 (segment (start 156.21 98.171) (end 155.956 97.917) (width 0.2) (layer "B.Cu") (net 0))
 (segment (start 153.035 99.695) (end 161.163 99.695) (width 0.2) (layer "B.Cu") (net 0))
 (segment (start 145.542 100.711) (end 144.653 100.711) (width 0.2) (layer "B.Cu") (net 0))
 (segment (start 173.101 97.536) (end 174.625 99.06) (width 0.2) (layer "B.Cu") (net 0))
 (segment (start 147.955 99.949) (end 149.225 101.219) (width 0.2) (layer "B.Cu") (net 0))
 (segment (start 153.924 100.838) (end 154.305 101.219) (width 0.2) (layer "B.Cu") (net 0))
 (segment (start 151.765 100.838) (end 153.924 100.838) (width 0.2) (layer "B.Cu") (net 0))
 (segment (start 154.305 101.219) (end 154.305 108.585) (width 0.2) (layer "B.Cu") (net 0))
 (segment (start 157.734 96.774) (end 176.657 96.774) (width 0.2) (layer "B.Cu") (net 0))
 (segment (start 144.653 100.711) (end 144.145 101.219) (width 0.2) (layer "B.Cu") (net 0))
 (segment (start 144.145 101.219) (end 144.145 108.585) (width 0.2) (layer "B.Cu") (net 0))
 (segment (start 167.005 99.568) (end 167.005 108.585) (width 0.2) (layer "B.Cu") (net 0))
 (segment (start 149.733 97.536) (end 149.733 98.806) (width 0.2) (layer "B.Cu") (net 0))
 (segment (start 163.957 99.314) (end 164.465 99.822) (width 0.2) (layer "B.Cu") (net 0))
 (segment (start 176.657 96.774) (end 177.419 97.536) (width 0.2) (layer "B.Cu") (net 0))
 (segment (start 151.511 97.536) (end 151.511 99.314) (width 0.2) (layer "B.Cu") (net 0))
 (segment (start 150.622 99.06) (end 152.019 100.457) (width 0.2) (layer "B.Cu") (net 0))
 (segment (start 177.419 108.331) (end 175.895 109.855) (width 0.2) (layer "B.Cu") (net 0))
 (segment (start 151.765 108.585) (end 150.495 109.855) (width 0.2) (layer "B.Cu") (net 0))
 (segment (start 154.178 98.552) (end 154.559 98.933) (width 0.2) (layer "B.Cu") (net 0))
 (segment (start 146.685 108.585) (end 145.415 109.855) (width 0.2) (layer "B.Cu") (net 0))
 (segment (start 151.765 101.6) (end 151.765 108.585) (width 0.2) (layer "B.Cu") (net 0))
 (segment (start 154.305 108.585) (end 153.035 109.855) (width 0.2) (layer "B.Cu") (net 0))
 (segment (start 166.37 98.933) (end 167.005 99.568) (width 0.2) (layer "B.Cu") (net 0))
 (segment (start 156.337 100.457) (end 156.845 100.965) (width 0.2) (layer "B.Cu") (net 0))
 (segment (start 154.178 97.536) (end 154.178 98.552) (width 0.2) (layer "B.Cu") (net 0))
 (segment (start 161.925 108.585) (end 160.655 109.855) (width 0.2) (layer "B.Cu") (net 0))
 (segment (start 153.289 97.536) (end 153.289 98.933) (width 0.2) (layer "B.Cu") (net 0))
 (segment (start 152.273 100.076) (end 158.623 100.076) (width 0.2) (layer "B.Cu") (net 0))
 (segment (start 155.067 98.298) (end 155.321 98.552) (width 0.2) (layer "B.Cu") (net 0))
 (segment (start 153.67 99.314) (end 163.957 99.314) (width 0.2) (layer "B.Cu") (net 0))
 (segment (start 148.844 98.679) (end 151.765 101.6) (width 0.2) (layer "B.Cu") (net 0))
 (segment (start 155.067 97.536) (end 155.067 98.298) (width 0.2) (layer "B.Cu") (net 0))
 (segment (start 147.066 101.219) (end 146.685 101.6) (width 0.2) (layer "B.Cu") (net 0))
 (segment (start 146.177 97.536) (end 146.177 100.076) (width 0.2) (layer "B.Cu") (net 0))
 (segment (start 148.844 97.536) (end 148.844 98.679) (width 0.2) (layer "B.Cu") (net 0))
 (segment (start 150.622 97.536) (end 150.622 99.06) (width 0.2) (layer "B.Cu") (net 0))
 (segment (start 152.019 100.457) (end 156.337 100.457) (width 0.2) (layer "B.Cu") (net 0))
 (segment (start 149.225 108.585) (end 147.955 109.855) (width 0.2) (layer "B.Cu") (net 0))
 (segment (start 156.845 108.585) (end 155.575 109.855) (width 0.2) (layer "B.Cu") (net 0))
 (segment (start 151.511 99.314) (end 152.273 100.076) (width 0.2) (layer "B.Cu") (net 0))
 (segment (start 169.545 108.585) (end 168.275 109.855) (width 0.2) (layer "B.Cu") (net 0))
 (segment (start 159.385 100.838) (end 159.385 108.585) (width 0.2) (layer "B.Cu") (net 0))
 (segment (start 153.289 98.933) (end 153.67 99.314) (width 0.2) (layer "B.Cu") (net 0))
 (segment (start 174.625 108.585) (end 173.355 109.855) (width 0.2) (layer "B.Cu") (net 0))
 (segment (start 168.783 98.552) (end 169.545 99.314) (width 0.2) (layer "B.Cu") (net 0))
 (segment (start 149.733 98.806) (end 151.765 100.838) (width 0.2) (layer "B.Cu") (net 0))
 (segment (start 154.559 98.933) (end 166.37 98.933) (width 0.2) (layer "B.Cu") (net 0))
 (segment (start 149.225 101.219) (end 149.225 108.585) (width 0.2) (layer "B.Cu") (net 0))
 (segment (start 155.956 97.917) (end 155.956 97.536) (width 0.2) (layer "B.Cu") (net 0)))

